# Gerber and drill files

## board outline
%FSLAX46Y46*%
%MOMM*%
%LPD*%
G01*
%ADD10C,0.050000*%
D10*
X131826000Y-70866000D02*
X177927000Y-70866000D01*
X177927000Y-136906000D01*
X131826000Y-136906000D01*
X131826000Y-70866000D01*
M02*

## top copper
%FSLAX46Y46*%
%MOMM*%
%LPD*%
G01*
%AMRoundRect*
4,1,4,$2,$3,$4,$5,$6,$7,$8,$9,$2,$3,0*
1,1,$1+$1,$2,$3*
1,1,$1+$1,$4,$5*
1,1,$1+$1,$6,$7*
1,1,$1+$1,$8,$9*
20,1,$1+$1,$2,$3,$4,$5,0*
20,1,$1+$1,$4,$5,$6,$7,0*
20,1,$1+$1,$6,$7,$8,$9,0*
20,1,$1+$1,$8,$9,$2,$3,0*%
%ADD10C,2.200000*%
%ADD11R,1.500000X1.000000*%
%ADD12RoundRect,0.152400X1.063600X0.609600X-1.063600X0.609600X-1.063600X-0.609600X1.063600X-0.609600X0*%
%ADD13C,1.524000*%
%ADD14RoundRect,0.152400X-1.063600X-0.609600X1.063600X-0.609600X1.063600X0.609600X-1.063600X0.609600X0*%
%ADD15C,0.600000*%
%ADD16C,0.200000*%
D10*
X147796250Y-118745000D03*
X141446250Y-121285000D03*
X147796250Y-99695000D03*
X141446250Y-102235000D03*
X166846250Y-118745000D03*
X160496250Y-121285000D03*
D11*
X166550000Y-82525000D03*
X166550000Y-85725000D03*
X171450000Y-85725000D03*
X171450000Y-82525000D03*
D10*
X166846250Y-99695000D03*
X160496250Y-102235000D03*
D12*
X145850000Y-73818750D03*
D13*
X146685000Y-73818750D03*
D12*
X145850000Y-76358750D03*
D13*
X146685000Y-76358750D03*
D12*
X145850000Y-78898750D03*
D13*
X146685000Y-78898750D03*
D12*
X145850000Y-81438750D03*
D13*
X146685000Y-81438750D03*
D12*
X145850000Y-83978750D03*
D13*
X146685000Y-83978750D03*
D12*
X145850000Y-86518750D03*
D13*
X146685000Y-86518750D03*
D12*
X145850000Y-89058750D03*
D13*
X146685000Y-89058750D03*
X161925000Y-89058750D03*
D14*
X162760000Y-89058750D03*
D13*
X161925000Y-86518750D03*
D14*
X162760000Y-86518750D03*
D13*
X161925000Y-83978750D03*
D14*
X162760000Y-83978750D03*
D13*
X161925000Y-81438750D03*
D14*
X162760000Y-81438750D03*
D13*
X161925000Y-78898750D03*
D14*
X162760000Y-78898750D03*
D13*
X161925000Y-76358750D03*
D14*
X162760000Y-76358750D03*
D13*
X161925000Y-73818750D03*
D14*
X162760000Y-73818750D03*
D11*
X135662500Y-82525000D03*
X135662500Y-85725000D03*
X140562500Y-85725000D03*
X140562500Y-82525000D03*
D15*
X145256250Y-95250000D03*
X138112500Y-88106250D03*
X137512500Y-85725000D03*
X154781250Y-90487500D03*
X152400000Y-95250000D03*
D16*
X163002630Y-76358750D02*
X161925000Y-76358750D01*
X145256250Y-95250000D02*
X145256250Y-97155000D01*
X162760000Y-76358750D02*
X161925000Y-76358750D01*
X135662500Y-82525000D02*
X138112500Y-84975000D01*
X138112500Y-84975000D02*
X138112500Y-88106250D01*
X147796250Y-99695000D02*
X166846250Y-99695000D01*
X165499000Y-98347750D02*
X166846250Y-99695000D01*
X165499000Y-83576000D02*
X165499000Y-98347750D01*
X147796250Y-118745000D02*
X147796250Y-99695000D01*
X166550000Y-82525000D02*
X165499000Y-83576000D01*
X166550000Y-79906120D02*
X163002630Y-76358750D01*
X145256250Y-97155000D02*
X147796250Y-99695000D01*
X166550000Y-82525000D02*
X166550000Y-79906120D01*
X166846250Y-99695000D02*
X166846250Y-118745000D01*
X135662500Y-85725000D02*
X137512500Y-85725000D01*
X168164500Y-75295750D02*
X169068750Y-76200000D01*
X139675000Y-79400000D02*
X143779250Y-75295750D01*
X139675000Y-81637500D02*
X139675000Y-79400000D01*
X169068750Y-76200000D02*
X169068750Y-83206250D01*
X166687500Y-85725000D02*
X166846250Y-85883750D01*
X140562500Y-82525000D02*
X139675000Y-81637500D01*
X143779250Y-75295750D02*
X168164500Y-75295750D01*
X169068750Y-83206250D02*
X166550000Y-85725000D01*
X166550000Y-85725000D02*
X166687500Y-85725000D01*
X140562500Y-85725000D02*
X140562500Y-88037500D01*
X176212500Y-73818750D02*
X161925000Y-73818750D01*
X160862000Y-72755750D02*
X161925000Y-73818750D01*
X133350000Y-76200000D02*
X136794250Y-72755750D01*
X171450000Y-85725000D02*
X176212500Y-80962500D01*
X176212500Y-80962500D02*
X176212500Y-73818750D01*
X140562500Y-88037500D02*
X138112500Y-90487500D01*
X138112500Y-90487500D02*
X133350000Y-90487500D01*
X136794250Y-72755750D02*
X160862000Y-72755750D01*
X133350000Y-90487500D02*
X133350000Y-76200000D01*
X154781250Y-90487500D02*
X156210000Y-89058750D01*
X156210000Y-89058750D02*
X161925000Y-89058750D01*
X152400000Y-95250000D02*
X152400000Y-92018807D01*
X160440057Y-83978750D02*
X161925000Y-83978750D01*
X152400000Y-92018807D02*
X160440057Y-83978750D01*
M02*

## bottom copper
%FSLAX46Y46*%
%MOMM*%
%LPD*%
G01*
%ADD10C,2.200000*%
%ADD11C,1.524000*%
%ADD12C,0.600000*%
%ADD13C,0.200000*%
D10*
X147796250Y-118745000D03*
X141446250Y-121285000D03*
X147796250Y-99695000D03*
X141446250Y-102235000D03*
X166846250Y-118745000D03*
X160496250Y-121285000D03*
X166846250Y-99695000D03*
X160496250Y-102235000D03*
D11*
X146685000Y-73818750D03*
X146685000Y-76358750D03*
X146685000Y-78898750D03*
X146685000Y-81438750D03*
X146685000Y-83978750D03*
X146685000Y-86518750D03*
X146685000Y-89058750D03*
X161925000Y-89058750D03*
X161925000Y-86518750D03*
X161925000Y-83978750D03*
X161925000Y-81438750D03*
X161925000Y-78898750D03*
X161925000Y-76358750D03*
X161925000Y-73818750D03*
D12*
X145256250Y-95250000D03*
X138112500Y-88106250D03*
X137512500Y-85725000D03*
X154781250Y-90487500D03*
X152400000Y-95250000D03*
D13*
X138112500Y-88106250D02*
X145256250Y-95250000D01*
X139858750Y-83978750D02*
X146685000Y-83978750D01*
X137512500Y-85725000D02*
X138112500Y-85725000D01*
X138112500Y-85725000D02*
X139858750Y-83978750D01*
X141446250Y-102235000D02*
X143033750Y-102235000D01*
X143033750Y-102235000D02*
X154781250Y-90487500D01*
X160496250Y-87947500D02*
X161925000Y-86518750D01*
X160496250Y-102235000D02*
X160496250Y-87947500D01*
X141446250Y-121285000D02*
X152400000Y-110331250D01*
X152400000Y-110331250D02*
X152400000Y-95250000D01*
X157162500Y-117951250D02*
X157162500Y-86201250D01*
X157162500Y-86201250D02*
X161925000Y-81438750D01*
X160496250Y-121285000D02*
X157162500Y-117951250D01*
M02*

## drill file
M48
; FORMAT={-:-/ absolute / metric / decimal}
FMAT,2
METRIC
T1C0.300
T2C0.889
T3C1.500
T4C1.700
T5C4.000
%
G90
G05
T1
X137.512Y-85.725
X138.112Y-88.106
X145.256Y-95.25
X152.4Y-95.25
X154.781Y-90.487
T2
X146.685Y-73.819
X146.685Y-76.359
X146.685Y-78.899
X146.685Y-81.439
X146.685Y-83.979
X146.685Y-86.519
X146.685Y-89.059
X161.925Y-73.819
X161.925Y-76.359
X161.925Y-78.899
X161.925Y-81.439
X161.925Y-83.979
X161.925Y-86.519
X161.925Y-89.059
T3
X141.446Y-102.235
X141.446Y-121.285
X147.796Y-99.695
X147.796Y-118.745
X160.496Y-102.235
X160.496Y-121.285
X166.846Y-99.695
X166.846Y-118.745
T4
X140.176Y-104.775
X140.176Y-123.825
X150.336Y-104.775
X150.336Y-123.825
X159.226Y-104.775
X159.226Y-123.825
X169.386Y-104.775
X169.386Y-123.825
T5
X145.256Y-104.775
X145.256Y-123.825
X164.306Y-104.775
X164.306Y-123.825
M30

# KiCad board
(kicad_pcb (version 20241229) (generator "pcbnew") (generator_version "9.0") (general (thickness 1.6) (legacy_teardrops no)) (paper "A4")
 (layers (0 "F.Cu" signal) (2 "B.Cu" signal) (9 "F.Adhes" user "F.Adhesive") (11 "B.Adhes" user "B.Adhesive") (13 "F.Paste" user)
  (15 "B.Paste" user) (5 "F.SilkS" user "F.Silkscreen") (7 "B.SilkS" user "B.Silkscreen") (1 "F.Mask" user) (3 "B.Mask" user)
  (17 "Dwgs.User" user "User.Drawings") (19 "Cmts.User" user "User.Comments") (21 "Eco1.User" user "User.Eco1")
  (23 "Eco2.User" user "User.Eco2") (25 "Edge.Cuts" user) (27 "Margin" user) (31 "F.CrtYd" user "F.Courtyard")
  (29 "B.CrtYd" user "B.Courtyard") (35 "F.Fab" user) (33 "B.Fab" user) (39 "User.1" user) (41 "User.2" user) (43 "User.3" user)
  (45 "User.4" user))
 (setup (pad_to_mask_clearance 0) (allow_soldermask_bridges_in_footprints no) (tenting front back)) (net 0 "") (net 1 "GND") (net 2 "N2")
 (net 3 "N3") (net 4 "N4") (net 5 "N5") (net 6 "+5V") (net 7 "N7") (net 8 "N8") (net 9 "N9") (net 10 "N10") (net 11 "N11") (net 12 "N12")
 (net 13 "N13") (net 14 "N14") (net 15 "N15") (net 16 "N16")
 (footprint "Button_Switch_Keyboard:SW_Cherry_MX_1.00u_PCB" (layer "F.Cu") (at 147.79625 118.745)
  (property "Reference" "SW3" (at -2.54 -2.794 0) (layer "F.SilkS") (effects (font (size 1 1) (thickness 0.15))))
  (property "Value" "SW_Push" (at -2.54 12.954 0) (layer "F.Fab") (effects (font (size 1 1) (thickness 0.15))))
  (pad "" np_thru_hole circle (at -7.62 5.08) (size 1.7 1.7) (drill 1.7) (layers "*.Cu" "*.Mask"))
  (pad "" np_thru_hole circle (at -2.54 5.08) (size 4 4) (drill 4) (layers "*.Cu" "*.Mask"))
  (pad "" np_thru_hole circle (at 2.54 5.08) (size 1.7 1.7) (drill 1.7) (layers "*.Cu" "*.Mask"))
  (pad "1" thru_hole circle (at 0 0) (size 2.2 2.2) (drill 1.5) (layers "*.Cu" "*.Mask") (remove_unused_layers no) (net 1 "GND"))
  (pad "2" thru_hole circle (at -6.35 2.54) (size 2.2 2.2) (drill 1.5) (layers "*.Cu" "*.Mask") (remove_unused_layers no) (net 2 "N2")))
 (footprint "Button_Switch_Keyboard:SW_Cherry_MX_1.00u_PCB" (layer "F.Cu") (at 147.79625 99.695)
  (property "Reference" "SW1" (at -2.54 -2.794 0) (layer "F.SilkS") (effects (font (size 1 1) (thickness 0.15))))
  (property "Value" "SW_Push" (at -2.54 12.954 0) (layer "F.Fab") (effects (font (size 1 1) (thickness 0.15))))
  (pad "" np_thru_hole circle (at -7.62 5.08) (size 1.7 1.7) (drill 1.7) (layers "*.Cu" "*.Mask"))
  (pad "" np_thru_hole circle (at -2.54 5.08) (size 4 4) (drill 4) (layers "*.Cu" "*.Mask"))
  (pad "" np_thru_hole circle (at 2.54 5.08) (size 1.7 1.7) (drill 1.7) (layers "*.Cu" "*.Mask"))
  (pad "1" thru_hole circle (at 0 0) (size 2.2 2.2) (drill 1.5) (layers "*.Cu" "*.Mask") (remove_unused_layers no) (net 1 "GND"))
  (pad "2" thru_hole circle (at -6.35 2.54) (size 2.2 2.2) (drill 1.5) (layers "*.Cu" "*.Mask") (remove_unused_layers no) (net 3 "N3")))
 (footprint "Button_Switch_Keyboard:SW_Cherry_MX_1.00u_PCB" (layer "F.Cu") (at 166.84625 118.745)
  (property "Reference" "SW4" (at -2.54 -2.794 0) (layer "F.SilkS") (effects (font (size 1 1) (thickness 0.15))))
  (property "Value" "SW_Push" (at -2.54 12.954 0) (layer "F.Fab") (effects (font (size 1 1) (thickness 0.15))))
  (pad "" np_thru_hole circle (at -7.62 5.08) (size 1.7 1.7) (drill 1.7) (layers "*.Cu" "*.Mask"))
  (pad "" np_thru_hole circle (at -2.54 5.08) (size 4 4) (drill 4) (layers "*.Cu" "*.Mask"))
  (pad "" np_thru_hole circle (at 2.54 5.08) (size 1.7 1.7) (drill 1.7) (layers "*.Cu" "*.Mask"))
  (pad "1" thru_hole circle (at 0 0) (size 2.2 2.2) (drill 1.5) (layers "*.Cu" "*.Mask") (remove_unused_layers no) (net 1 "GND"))
  (pad "2" thru_hole circle (at -6.35 2.54) (size 2.2 2.2) (drill 1.5) (layers "*.Cu" "*.Mask") (remove_unused_layers no) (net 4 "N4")))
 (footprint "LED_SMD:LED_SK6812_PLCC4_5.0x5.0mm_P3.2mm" (layer "F.Cu") (at 169 84.125)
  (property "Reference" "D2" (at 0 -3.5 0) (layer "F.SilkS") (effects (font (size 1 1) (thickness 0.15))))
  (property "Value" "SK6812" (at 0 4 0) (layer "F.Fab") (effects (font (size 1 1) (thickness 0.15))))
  (pad "1" smd rect (at -2.45 -1.6 180) (size 1.5 1) (layers "F.Cu" "F.Mask" "F.Paste") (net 1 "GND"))
  (pad "2" smd rect (at -2.45 1.6 180) (size 1.5 1) (layers "F.Cu" "F.Mask" "F.Paste") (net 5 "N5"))
  (pad "3" smd rect (at 2.45 1.6 180) (size 1.5 1) (layers "F.Cu" "F.Mask" "F.Paste") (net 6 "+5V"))
  (pad "4" smd rect (at 2.45 -1.6 180) (size 1.5 1) (layers "F.Cu" "F.Mask" "F.Paste") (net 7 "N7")))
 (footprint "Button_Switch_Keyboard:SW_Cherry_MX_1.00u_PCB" (layer "F.Cu") (at 166.84625 99.695)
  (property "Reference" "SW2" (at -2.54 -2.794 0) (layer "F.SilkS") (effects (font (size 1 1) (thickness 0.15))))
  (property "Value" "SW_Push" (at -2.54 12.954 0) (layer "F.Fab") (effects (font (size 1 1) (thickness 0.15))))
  (pad "" np_thru_hole circle (at -7.62 5.08) (size 1.7 1.7) (drill 1.7) (layers "*.Cu" "*.Mask"))
  (pad "" np_thru_hole circle (at -2.54 5.08) (size 4 4) (drill 4) (layers "*.Cu" "*.Mask"))
  (pad "" np_thru_hole circle (at 2.54 5.08) (size 1.7 1.7) (drill 1.7) (layers "*.Cu" "*.Mask"))
  (pad "1" thru_hole circle (at 0 0) (size 2.2 2.2) (drill 1.5) (layers "*.Cu" "*.Mask") (remove_unused_layers no) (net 1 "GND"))
  (pad "2" thru_hole circle (at -6.35 2.54) (size 2.2 2.2) (drill 1.5) (layers "*.Cu" "*.Mask") (remove_unused_layers no) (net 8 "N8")))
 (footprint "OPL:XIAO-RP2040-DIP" (layer "F.Cu") (at 154.305 81.43875)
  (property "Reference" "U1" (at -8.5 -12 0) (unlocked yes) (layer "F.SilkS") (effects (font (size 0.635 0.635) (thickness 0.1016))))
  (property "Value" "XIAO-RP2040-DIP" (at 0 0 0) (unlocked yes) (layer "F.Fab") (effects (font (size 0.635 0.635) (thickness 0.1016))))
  (pad "1" smd roundrect (at -8.455 -7.62 180) (size 2.432 1.524) (layers "F.Cu" "F.Mask") (roundrect_rratio 0.1) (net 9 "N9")
   (thermal_bridge_angle 45))
  (pad "1" thru_hole circle (at -7.62 -7.62 180) (size 1.524 1.524) (drill 0.889) (layers "*.Cu" "*.Mask") (remove_unused_layers no)
   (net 9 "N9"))
  (pad "2" smd roundrect (at -8.455 -5.08 180) (size 2.432 1.524) (layers "F.Cu" "F.Mask") (roundrect_rratio 0.1) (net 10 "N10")
   (thermal_bridge_angle 45))
  (pad "2" thru_hole circle (at -7.62 -5.08 180) (size 1.524 1.524) (drill 0.889) (layers "*.Cu" "*.Mask") (remove_unused_layers no)
   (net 10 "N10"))
  (pad "3" smd roundrect (at -8.455 -2.54 180) (size 2.432 1.524) (layers "F.Cu" "F.Mask") (roundrect_rratio 0.1) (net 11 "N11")
   (thermal_bridge_angle 45))
  (pad "3" thru_hole circle (at -7.62 -2.54 180) (size 1.524 1.524) (drill 0.889) (layers "*.Cu" "*.Mask") (remove_unused_layers no)
   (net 11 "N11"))
  (pad "4" smd roundrect (at -8.455 0 180) (size 2.432 1.524) (layers "F.Cu" "F.Mask") (roundrect_rratio 0.1) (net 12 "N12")
   (thermal_bridge_angle 45))
  (pad "4" thru_hole circle (at -7.62 0 180) (size 1.524 1.524) (drill 0.889) (layers "*.Cu" "*.Mask") (remove_unused_layers no)
   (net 12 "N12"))
  (pad "5" smd roundrect (at -8.455 2.54 180) (size 2.432 1.524) (layers "F.Cu" "F.Mask") (roundrect_rratio 0.1) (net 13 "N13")
   (thermal_bridge_angle 45))
  (pad "5" thru_hole circle (at -7.62 2.54 180) (size 1.524 1.524) (drill 0.889) (layers "*.Cu" "*.Mask") (remove_unused_layers no)
   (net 13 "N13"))
  (pad "6" smd roundrect (at -8.455 5.08 180) (size 2.432 1.524) (layers "F.Cu" "F.Mask") (roundrect_rratio 0.1) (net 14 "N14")
   (thermal_bridge_angle 45))
  (pad "6" thru_hole circle (at -7.62 5.08 180) (size 1.524 1.524) (drill 0.889) (layers "*.Cu" "*.Mask") (remove_unused_layers no)
   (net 14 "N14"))
  (pad "7" smd roundrect (at -8.455 7.62 180) (size 2.432 1.524) (layers "F.Cu" "F.Mask") (roundrect_rratio 0.1) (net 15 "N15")
   (thermal_bridge_angle 45))
  (pad "7" thru_hole circle (at -7.62 7.62 180) (size 1.524 1.524) (drill 0.889) (layers "*.Cu" "*.Mask") (remove_unused_layers no)
   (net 15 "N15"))
  (pad "8" thru_hole circle (at 7.62 7.62) (size 1.524 1.524) (drill 0.889) (layers "*.Cu" "*.Mask") (remove_unused_layers no) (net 3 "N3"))
  (pad "8" smd roundrect (at 8.455 7.62) (size 2.432 1.524) (layers "F.Cu" "F.Mask") (roundrect_rratio 0.1) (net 3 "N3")
   (thermal_bridge_angle 45))
  (pad "9" thru_hole circle (at 7.62 5.08) (size 1.524 1.524) (drill 0.889) (layers "*.Cu" "*.Mask") (remove_unused_layers no) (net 8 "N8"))
  (pad "9" smd roundrect (at 8.455 5.08) (size 2.432 1.524) (layers "F.Cu" "F.Mask") (roundrect_rratio 0.1) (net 8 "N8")
   (thermal_bridge_angle 45))
  (pad "10" thru_hole circle (at 7.62 2.54) (size 1.524 1.524) (drill 0.889) (layers "*.Cu" "*.Mask") (remove_unused_layers no) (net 2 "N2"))
  (pad "10" smd roundrect (at 8.455 2.54) (size 2.432 1.524) (layers "F.Cu" "F.Mask") (roundrect_rratio 0.1) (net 2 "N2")
   (thermal_bridge_angle 45))
  (pad "11" thru_hole circle (at 7.62 0) (size 1.524 1.524) (drill 0.889) (layers "*.Cu" "*.Mask") (remove_unused_layers no) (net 4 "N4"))
  (pad "11" smd roundrect (at 8.455 0) (size 2.432 1.524) (layers "F.Cu" "F.Mask") (roundrect_rratio 0.1) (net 4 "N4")
   (thermal_bridge_angle 45))
  (pad "12" thru_hole circle (at 7.62 -2.54) (size 1.524 1.524) (drill 0.889) (layers "*.Cu" "*.Mask") (remove_unused_layers no)
   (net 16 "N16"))
  (pad "12" smd roundrect (at 8.455 -2.54) (size 2.432 1.524) (layers "F.Cu" "F.Mask") (roundrect_rratio 0.1) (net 16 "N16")
   (thermal_bridge_angle 45))
  (pad "13" thru_hole circle (at 7.62 -5.08) (size 1.524 1.524) (drill 0.889) (layers "*.Cu" "*.Mask") (remove_unused_layers no)
   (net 1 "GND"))
  (pad "13" smd roundrect (at 8.455 -5.08) (size 2.432 1.524) (layers "F.Cu" "F.Mask") (roundrect_rratio 0.1) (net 1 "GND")
   (thermal_bridge_angle 45))
  (pad "14" thru_hole circle (at 7.62 -7.62) (size 1.524 1.524) (drill 0.889) (layers "*.Cu" "*.Mask") (remove_unused_layers no)
   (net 6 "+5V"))
  (pad "14" smd roundrect (at 8.455 -7.62) (size 2.432 1.524) (layers "F.Cu" "F.Mask") (roundrect_rratio 0.1) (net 6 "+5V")
   (thermal_bridge_angle 45)))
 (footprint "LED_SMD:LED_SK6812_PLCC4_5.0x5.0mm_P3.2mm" (layer "F.Cu") (at 138.1125 84.125)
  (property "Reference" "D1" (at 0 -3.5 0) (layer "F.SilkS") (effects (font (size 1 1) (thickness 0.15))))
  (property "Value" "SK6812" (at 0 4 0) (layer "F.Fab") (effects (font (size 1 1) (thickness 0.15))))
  (pad "1" smd rect (at -2.45 -1.6 180) (size 1.5 1) (layers "F.Cu" "F.Mask" "F.Paste") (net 1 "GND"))
  (pad "2" smd rect (at -2.45 1.6 180) (size 1.5 1) (layers "F.Cu" "F.Mask" "F.Paste") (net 13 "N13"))
  (pad "3" smd rect (at 2.45 1.6 180) (size 1.5 1) (layers "F.Cu" "F.Mask" "F.Paste") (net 6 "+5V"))
  (pad "4" smd rect (at 2.45 -1.6 180) (size 1.5 1) (layers "F.Cu" "F.Mask" "F.Paste") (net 5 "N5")))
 (gr_rect (start 131.826 70.866) (end 177.927 136.906) (stroke (width 0.05) (type default)) (fill no) (layer "Edge.Cuts"))
 (segment (start 163.00263 76.35875) (end 161.925 76.35875) (width 0.2) (layer "F.Cu") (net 1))
 (segment (start 145.25625 95.25) (end 145.25625 97.155) (width 0.2) (layer "F.Cu") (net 1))
 (segment (start 162.76 76.35875) (end 161.925 76.35875) (width 0.2) (layer "F.Cu") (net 1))
 (segment (start 135.6625 82.525) (end 138.1125 84.975) (width 0.2) (layer "F.Cu") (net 1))
 (segment (start 138.1125 84.975) (end 138.1125 88.10625) (width 0.2) (layer "F.Cu") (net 1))
 (segment (start 147.79625 99.695) (end 166.84625 99.695) (width 0.2) (layer "F.Cu") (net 1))
 (segment (start 165.499 98.34775) (end 166.84625 99.695) (width 0.2) (layer "F.Cu") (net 1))
 (segment (start 165.499 83.576) (end 165.499 98.34775) (width 0.2) (layer "F.Cu") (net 1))
 (segment (start 147.79625 118.745) (end 147.79625 99.695) (width 0.2) (layer "F.Cu") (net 1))
 (segment (start 166.55 82.525) (end 165.499 83.576) (width 0.2) (layer "F.Cu") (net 1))
 (segment (start 166.55 79.90612) (end 163.00263 76.35875) (width 0.2) (layer "F.Cu") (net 1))
 (segment (start 145.25625 97.155) (end 147.79625 99.695) (width 0.2) (layer "F.Cu") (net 1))
 (segment (start 166.55 82.525) (end 166.55 79.90612) (width 0.2) (layer "F.Cu") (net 1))
 (segment (start 166.84625 99.695) (end 166.84625 118.745) (width 0.2) (layer "F.Cu") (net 1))
 (via (at 145.25625 95.25) (size 0.6) (drill 0.3) (layers "F.Cu" "B.Cu") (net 1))
 (via (at 138.1125 88.10625) (size 0.6) (drill 0.3) (layers "F.Cu" "B.Cu") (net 1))
 (segment (start 138.1125 88.10625) (end 145.25625 95.25) (width 0.2) (layer "B.Cu") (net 1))
 (segment (start 135.6625 85.725) (end 137.5125 85.725) (width 0.2) (layer "F.Cu") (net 13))
 (via (at 137.5125 85.725) (size 0.6) (drill 0.3) (layers "F.Cu" "B.Cu") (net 13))
 (segment (start 139.85875 83.97875) (end 146.685 83.97875) (width 0.2) (layer "B.Cu") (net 13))
 (segment (start 137.5125 85.725) (end 138.1125 85.725) (width 0.2) (layer "B.Cu") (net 13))
 (segment (start 138.1125 85.725) (end 139.85875 83.97875) (width 0.2) (layer "B.Cu") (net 13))
 (segment (start 168.1645 75.29575) (end 169.06875 76.2) (width 0.2) (layer "F.Cu") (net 5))
 (segment (start 139.675 79.4) (end 143.77925 75.29575) (width 0.2) (layer "F.Cu") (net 5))
 (segment (start 139.675 81.6375) (end 139.675 79.4) (width 0.2) (layer "F.Cu") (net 5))
 (segment (start 169.06875 76.2) (end 169.06875 83.20625) (width 0.2) (layer "F.Cu") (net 5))
 (segment (start 166.6875 85.725) (end 166.84625 85.88375) (width 0.2) (layer "F.Cu") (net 5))
 (segment (start 140.5625 82.525) (end 139.675 81.6375) (width 0.2) (layer "F.Cu") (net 5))
 (segment (start 143.77925 75.29575) (end 168.1645 75.29575) (width 0.2) (layer "F.Cu") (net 5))
 (segment (start 169.06875 83.20625) (end 166.55 85.725) (width 0.2) (layer "F.Cu") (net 5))
 (segment (start 166.55 85.725) (end 166.6875 85.725) (width 0.2) (layer "F.Cu") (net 5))
 (segment (start 140.5625 85.725) (end 140.5625 88.0375) (width 0.2) (layer "F.Cu") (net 6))
 (segment (start 176.2125 73.81875) (end 161.925 73.81875) (width 0.2) (layer "F.Cu") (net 6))
 (segment (start 160.862 72.75575) (end 161.925 73.81875) (width 0.2) (layer "F.Cu") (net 6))
 (segment (start 133.35 76.2) (end 136.79425 72.75575) (width 0.2) (layer "F.Cu") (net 6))
 (segment (start 171.45 85.725) (end 176.2125 80.9625) (width 0.2) (layer "F.Cu") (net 6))
 (segment (start 176.2125 80.9625) (end 176.2125 73.81875) (width 0.2) (layer "F.Cu") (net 6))
 (segment (start 140.5625 88.0375) (end 138.1125 90.4875) (width 0.2) (layer "F.Cu") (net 6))
 (segment (start 138.1125 90.4875) (end 133.35 90.4875) (width 0.2) (layer "F.Cu") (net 6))
 (segment (start 136.79425 72.75575) (end 160.862 72.75575) (width 0.2) (layer "F.Cu") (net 6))
 (segment (start 133.35 90.4875) (end 133.35 76.2) (width 0.2) (layer "F.Cu") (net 6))
 (segment (start 154.78125 90.4875) (end 156.21 89.05875) (width 0.2) (layer "F.Cu") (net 3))
 (segment (start 156.21 89.05875) (end 161.925 89.05875) (width 0.2) (layer "F.Cu") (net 3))
 (via (at 154.78125 90.4875) (size 0.6) (drill 0.3) (layers "F.Cu" "B.Cu") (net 3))
 (segment (start 141.44625 102.235) (end 143.03375 102.235) (width 0.2) (layer "B.Cu") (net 3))
 (segment (start 143.03375 102.235) (end 154.78125 90.4875) (width 0.2) (layer "B.Cu") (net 3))
 (segment (start 160.49625 87.9475) (end 161.925 86.51875) (width 0.2) (layer "B.Cu") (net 8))
 (segment (start 160.49625 102.235) (end 160.49625 87.9475) (width 0.2) (layer "B.Cu") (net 8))
 (segment (start 152.4 95.25) (end 152.4 92.018807) (width 0.2) (layer "F.Cu") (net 2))
 (segment (start 160.440057 83.97875) (end 161.925 83.97875) (width 0.2) (layer "F.Cu") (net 2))
 (segment (start 152.4 92.018807) (end 160.440057 83.97875) (width 0.2) (layer "F.Cu") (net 2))
 (via (at 152.4 95.25) (size 0.6) (drill 0.3) (layers "F.Cu" "B.Cu") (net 2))
 (segment (start 141.44625 121.285) (end 152.4 110.33125) (width 0.2) (layer "B.Cu") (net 2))
 (segment (start 152.4 110.33125) (end 152.4 95.25) (width 0.2) (layer "B.Cu") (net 2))
 (segment (start 157.1625 117.95125) (end 157.1625 86.20125) (width 0.2) (layer "B.Cu") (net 4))
 (segment (start 157.1625 86.20125) (end 161.925 81.43875) (width 0.2) (layer "B.Cu") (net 4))
 (segment (start 160.49625 121.285) (end 157.1625 117.95125) (width 0.2) (layer "B.Cu") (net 4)))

